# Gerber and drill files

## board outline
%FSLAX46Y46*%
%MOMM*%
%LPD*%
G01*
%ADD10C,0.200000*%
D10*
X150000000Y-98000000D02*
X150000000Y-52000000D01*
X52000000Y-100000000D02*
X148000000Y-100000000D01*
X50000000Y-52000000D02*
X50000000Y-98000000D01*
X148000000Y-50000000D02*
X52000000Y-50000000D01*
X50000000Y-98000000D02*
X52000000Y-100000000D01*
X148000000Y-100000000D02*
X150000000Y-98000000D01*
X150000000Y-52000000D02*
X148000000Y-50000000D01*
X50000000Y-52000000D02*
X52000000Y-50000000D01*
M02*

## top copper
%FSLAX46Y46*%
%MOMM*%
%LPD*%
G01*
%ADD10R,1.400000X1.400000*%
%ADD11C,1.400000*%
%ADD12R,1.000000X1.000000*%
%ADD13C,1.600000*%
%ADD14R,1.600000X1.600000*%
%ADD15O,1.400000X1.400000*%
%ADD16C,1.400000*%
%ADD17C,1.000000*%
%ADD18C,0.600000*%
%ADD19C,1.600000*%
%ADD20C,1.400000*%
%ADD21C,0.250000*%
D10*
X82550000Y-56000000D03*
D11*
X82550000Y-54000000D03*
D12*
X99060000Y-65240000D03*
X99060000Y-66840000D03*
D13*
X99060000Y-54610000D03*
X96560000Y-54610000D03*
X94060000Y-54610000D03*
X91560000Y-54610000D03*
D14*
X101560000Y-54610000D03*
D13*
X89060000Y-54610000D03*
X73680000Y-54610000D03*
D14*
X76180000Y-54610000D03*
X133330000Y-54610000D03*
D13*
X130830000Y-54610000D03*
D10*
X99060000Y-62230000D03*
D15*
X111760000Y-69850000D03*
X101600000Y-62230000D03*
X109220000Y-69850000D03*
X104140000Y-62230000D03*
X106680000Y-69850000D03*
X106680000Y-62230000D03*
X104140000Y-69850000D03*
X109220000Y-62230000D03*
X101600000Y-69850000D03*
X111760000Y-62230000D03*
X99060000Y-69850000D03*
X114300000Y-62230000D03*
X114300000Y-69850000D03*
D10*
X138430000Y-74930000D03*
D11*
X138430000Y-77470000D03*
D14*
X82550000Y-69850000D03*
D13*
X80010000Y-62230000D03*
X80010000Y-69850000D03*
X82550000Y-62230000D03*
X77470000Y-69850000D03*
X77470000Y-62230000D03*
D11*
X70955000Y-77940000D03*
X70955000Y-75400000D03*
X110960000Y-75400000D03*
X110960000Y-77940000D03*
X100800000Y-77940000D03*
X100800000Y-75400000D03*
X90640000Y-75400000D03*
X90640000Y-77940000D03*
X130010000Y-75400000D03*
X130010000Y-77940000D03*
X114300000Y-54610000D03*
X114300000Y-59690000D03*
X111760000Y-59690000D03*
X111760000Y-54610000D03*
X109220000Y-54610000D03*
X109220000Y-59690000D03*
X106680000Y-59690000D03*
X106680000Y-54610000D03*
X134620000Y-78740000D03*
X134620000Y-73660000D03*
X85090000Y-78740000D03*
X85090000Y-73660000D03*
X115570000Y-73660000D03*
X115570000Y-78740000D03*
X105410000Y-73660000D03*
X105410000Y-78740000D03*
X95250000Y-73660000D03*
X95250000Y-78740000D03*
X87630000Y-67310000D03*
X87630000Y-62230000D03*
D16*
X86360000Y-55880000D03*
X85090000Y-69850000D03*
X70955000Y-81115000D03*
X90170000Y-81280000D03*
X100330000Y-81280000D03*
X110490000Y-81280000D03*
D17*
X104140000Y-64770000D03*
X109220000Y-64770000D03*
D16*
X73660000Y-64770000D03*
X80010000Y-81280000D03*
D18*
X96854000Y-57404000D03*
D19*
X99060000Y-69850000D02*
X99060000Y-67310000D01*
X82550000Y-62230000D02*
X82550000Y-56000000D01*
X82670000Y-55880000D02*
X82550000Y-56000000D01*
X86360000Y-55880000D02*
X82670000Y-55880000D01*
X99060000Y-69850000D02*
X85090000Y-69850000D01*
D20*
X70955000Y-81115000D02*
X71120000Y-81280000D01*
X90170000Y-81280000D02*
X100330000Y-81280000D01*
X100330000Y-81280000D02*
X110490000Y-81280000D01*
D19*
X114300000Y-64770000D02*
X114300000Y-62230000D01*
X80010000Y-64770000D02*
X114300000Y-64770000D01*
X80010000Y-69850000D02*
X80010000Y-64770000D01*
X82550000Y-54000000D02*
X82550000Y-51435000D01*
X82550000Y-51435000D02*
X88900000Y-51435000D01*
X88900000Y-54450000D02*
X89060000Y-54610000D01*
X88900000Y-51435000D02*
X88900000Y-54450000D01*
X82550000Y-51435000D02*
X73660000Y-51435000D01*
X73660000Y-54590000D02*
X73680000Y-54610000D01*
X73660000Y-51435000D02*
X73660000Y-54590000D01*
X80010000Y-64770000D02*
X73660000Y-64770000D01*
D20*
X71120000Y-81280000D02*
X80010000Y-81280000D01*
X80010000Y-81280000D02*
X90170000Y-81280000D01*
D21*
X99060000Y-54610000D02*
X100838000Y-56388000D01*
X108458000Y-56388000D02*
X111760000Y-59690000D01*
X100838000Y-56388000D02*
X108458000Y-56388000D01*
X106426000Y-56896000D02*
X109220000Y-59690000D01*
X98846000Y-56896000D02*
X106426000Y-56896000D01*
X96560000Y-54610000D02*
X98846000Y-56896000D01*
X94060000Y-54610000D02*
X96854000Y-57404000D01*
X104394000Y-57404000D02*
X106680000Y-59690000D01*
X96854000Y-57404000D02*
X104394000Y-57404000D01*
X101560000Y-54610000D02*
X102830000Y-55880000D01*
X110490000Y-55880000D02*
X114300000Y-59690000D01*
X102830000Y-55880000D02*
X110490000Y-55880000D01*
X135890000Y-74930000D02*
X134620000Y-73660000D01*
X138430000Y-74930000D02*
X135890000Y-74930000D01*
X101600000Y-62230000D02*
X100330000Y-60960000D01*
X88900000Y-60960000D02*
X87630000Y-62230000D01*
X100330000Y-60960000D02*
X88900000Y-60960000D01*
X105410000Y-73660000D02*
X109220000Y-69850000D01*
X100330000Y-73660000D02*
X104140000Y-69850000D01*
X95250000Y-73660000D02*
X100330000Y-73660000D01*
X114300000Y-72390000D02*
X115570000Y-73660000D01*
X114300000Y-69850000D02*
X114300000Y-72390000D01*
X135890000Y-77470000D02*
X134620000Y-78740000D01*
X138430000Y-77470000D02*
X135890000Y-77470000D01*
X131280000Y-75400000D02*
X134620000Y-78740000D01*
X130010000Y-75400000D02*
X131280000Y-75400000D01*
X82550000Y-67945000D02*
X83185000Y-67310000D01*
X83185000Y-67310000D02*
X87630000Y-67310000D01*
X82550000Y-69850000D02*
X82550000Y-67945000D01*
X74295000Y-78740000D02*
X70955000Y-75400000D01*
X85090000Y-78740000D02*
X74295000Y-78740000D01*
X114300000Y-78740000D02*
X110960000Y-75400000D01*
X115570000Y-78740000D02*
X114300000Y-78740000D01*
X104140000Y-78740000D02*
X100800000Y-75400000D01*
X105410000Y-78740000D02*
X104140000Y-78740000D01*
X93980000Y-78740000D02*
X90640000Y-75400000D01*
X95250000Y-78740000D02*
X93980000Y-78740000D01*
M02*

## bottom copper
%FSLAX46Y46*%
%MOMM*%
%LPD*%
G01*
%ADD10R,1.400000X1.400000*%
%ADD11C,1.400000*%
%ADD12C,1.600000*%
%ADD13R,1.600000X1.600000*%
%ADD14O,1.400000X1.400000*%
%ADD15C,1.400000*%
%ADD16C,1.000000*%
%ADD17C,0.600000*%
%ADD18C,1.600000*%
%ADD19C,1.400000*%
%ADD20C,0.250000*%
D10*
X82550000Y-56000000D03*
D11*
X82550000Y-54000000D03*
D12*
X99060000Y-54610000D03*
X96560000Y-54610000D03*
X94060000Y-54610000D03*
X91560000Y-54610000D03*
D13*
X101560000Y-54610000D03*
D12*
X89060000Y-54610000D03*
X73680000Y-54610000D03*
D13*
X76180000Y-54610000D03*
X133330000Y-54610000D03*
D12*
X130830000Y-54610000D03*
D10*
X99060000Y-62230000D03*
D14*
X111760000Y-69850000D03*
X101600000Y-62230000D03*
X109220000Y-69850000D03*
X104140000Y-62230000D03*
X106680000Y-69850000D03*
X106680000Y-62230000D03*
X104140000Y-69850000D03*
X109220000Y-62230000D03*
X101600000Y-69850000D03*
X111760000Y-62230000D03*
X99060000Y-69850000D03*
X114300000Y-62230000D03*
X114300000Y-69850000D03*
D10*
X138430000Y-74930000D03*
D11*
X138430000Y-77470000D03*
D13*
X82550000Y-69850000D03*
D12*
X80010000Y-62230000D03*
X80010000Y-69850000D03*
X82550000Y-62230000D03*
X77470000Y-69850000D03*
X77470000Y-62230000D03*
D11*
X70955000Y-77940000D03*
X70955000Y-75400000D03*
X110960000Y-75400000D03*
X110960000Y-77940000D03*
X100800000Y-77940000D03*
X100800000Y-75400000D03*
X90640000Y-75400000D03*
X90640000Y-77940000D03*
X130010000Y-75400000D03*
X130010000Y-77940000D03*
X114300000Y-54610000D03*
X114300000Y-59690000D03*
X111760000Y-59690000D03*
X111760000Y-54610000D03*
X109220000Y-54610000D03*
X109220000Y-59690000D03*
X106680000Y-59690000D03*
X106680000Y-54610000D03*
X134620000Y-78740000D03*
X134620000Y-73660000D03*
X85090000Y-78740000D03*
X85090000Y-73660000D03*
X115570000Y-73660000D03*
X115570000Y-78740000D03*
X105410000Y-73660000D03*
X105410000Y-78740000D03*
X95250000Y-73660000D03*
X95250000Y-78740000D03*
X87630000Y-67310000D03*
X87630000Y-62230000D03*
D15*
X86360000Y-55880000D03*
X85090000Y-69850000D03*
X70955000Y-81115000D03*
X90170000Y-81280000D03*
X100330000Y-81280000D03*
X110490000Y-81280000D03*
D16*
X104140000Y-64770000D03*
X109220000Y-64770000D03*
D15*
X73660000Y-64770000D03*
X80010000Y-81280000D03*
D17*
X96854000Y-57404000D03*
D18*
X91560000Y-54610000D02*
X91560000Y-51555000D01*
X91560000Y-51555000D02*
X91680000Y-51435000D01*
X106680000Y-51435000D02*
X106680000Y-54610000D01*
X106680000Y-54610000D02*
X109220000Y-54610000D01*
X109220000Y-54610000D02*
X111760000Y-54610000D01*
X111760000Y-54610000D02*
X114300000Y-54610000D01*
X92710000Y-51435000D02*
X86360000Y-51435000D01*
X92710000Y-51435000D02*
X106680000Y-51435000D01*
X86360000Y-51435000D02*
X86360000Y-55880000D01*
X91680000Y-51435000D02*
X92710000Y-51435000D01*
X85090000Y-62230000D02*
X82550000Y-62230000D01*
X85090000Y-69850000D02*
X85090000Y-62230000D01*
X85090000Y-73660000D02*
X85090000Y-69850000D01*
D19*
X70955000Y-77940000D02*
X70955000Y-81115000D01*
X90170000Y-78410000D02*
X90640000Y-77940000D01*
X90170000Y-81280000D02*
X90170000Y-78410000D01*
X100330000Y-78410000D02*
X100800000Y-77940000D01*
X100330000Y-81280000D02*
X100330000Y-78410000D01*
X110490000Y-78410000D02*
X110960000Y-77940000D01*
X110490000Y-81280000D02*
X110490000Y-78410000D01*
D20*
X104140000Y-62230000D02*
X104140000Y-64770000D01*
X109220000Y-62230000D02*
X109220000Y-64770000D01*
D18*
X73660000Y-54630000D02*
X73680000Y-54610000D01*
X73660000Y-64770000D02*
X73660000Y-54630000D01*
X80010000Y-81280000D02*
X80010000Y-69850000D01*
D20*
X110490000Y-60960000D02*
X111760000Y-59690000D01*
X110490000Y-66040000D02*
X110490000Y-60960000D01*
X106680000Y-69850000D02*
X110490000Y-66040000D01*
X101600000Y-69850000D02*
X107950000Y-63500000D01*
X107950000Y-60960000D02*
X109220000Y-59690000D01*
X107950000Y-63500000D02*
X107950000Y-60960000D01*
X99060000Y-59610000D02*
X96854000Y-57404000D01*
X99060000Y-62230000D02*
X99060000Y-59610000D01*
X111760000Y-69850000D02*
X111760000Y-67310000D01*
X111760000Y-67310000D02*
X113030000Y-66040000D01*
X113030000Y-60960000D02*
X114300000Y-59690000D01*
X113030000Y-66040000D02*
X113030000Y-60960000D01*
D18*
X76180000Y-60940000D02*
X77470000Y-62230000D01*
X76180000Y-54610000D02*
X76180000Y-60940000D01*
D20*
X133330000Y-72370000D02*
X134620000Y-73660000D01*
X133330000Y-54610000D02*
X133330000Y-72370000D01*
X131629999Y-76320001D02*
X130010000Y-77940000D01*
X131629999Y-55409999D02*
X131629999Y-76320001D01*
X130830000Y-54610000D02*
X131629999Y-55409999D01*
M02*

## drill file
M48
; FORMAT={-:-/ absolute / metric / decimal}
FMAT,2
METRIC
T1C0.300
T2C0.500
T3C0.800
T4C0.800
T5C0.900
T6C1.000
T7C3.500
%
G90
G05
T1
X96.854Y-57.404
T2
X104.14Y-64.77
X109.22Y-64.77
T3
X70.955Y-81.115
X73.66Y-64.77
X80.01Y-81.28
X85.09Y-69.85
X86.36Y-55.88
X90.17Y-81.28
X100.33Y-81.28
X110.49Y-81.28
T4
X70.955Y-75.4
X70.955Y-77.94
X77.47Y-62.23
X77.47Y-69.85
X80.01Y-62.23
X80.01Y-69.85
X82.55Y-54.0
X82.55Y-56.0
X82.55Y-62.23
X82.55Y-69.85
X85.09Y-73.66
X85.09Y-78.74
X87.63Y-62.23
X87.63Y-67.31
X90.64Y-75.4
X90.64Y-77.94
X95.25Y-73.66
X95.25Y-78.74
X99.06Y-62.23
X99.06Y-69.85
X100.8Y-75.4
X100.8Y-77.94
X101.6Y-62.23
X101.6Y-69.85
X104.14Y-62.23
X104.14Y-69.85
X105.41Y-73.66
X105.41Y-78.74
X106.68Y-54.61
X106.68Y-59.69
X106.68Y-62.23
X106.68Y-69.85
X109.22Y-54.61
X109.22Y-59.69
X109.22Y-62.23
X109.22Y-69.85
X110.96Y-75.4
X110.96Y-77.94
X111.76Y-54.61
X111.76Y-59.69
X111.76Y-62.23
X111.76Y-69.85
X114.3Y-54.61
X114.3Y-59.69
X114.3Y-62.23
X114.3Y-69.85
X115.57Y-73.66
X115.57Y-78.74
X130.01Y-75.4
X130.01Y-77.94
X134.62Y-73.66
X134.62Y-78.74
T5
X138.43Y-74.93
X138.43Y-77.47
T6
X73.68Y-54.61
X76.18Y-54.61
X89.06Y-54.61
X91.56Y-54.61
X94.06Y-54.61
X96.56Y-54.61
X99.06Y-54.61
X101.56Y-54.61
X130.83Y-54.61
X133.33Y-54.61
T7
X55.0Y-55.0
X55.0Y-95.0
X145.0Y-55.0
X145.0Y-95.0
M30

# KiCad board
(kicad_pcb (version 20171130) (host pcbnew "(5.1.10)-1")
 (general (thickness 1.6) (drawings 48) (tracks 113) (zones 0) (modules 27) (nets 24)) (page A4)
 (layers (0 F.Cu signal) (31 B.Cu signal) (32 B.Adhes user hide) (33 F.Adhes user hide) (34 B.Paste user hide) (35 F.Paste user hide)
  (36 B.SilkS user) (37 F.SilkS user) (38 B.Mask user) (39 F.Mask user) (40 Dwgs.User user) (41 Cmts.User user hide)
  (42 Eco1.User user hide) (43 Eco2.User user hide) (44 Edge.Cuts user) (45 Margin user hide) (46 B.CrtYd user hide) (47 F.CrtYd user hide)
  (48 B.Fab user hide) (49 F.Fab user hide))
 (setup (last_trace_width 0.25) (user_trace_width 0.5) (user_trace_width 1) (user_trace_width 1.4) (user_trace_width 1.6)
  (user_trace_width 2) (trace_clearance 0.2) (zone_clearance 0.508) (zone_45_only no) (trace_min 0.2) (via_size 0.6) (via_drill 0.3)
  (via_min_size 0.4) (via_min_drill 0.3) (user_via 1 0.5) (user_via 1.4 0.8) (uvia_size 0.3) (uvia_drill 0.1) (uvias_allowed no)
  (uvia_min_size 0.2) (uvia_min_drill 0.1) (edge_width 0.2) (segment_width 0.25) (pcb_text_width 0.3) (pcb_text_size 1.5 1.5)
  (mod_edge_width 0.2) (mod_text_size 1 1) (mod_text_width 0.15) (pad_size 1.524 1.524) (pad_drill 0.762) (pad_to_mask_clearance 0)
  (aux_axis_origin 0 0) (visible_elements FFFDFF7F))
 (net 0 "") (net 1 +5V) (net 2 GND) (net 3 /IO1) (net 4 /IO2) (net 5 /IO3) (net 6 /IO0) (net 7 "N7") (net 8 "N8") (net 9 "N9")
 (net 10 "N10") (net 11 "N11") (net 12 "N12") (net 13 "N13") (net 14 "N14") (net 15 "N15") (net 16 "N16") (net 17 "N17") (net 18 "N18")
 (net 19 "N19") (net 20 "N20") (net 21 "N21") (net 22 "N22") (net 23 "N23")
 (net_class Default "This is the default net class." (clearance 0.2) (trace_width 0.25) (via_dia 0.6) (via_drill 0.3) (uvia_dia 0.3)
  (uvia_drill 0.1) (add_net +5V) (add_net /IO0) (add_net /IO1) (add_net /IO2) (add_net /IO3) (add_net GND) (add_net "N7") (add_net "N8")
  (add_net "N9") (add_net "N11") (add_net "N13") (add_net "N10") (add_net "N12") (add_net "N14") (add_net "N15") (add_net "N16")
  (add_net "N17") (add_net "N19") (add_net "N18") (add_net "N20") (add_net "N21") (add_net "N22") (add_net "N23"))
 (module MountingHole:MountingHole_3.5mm (layer F.Cu) (at 145 55)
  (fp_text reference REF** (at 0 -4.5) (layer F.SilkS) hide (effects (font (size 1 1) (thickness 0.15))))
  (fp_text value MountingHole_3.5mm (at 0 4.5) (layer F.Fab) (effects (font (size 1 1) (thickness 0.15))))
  (pad 1 np_thru_hole circle (at 0 0) (size 3.5 3.5) (drill 3.5) (layers *.Cu *.Mask)))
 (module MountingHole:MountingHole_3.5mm (layer F.Cu) (at 145 95)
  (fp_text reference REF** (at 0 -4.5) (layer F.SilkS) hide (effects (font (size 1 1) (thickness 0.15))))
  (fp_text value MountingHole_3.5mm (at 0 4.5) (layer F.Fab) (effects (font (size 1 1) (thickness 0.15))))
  (pad 1 np_thru_hole circle (at 0 0) (size 3.5 3.5) (drill 3.5) (layers *.Cu *.Mask)))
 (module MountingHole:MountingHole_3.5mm (layer F.Cu) (at 55 95)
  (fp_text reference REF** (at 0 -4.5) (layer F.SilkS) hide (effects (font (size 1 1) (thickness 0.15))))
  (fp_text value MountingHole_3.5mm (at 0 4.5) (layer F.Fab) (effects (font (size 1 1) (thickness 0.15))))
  (pad 1 np_thru_hole circle (at 0 0) (size 3.5 3.5) (drill 3.5) (layers *.Cu *.Mask)))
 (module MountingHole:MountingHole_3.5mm (layer F.Cu) (at 55 55)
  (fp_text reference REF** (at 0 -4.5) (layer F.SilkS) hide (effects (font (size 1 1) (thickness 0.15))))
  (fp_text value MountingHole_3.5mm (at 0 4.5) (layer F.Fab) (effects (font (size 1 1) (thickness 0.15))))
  (pad 1 np_thru_hole circle (at 0 0) (size 3.5 3.5) (drill 3.5) (layers *.Cu *.Mask)))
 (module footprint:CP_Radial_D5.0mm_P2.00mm (layer B.Cu) (at 82.55 56 90)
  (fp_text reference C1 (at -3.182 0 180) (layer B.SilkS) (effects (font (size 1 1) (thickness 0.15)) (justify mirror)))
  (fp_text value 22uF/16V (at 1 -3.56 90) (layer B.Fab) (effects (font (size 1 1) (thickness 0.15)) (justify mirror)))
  (pad 1 thru_hole rect (at 0 0 90) (size 1.4 1.4) (drill 0.8) (layers *.Cu *.Mask) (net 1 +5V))
  (pad 2 thru_hole circle (at 2 0 90) (size 1.4 1.4) (drill 0.8) (layers *.Cu *.Mask) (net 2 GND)))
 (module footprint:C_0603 (layer F.Cu) (at 99.06 66.04 270)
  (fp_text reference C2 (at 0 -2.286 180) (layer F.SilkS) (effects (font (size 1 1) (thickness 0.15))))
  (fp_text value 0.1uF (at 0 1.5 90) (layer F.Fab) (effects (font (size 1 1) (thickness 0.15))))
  (pad 1 smd rect (at -0.8 0 270) (size 1 1) (layers F.Cu F.Paste F.Mask) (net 2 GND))
  (pad 2 smd rect (at 0.8 0 270) (size 1 1) (layers F.Cu F.Paste F.Mask) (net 1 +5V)))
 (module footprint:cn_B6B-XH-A (layer B.Cu) (at 95.31 54.61 180)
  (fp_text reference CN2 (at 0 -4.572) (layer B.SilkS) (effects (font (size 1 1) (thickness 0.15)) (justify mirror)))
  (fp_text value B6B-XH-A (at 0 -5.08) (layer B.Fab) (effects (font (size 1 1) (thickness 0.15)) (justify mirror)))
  (pad 2 thru_hole circle (at -3.75 0 180) (size 1.6 1.6) (drill 1) (layers *.Cu *.Mask) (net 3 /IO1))
  (pad 3 thru_hole circle (at -1.25 0 180) (size 1.6 1.6) (drill 1) (layers *.Cu *.Mask) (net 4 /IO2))
  (pad 4 thru_hole circle (at 1.25 0 180) (size 1.6 1.6) (drill 1) (layers *.Cu *.Mask) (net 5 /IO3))
  (pad 5 thru_hole circle (at 3.75 0 180) (size 1.6 1.6) (drill 1) (layers *.Cu *.Mask) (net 1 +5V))
  (pad 1 thru_hole rect (at -6.25 0 180) (size 1.6 1.6) (drill 1) (layers *.Cu *.Mask) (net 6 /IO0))
  (pad 6 thru_hole circle (at 6.25 0 180) (size 1.6 1.6) (drill 1) (layers *.Cu *.Mask) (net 2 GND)))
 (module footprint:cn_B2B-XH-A (layer B.Cu) (at 74.93 54.61 180)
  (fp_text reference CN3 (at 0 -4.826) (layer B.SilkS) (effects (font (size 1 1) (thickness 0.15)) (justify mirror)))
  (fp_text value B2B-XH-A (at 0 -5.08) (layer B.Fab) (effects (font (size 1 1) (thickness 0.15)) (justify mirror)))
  (pad 2 thru_hole circle (at 1.25 0 180) (size 1.6 1.6) (drill 1) (layers *.Cu *.Mask) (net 2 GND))
  (pad 1 thru_hole rect (at -1.25 0 180) (size 1.6 1.6) (drill 1) (layers *.Cu *.Mask) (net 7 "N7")))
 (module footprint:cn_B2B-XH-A (layer B.Cu) (at 132.08 54.61 180)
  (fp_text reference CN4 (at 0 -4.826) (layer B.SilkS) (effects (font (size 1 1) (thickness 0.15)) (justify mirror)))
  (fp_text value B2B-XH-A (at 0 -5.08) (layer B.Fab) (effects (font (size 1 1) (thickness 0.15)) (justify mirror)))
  (pad 1 thru_hole rect (at -1.25 0 180) (size 1.6 1.6) (drill 1) (layers *.Cu *.Mask) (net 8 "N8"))
  (pad 2 thru_hole circle (at 1.25 0 180) (size 1.6 1.6) (drill 1) (layers *.Cu *.Mask) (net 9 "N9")))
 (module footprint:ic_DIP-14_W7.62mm (layer B.Cu) (at 99.06 62.23 270)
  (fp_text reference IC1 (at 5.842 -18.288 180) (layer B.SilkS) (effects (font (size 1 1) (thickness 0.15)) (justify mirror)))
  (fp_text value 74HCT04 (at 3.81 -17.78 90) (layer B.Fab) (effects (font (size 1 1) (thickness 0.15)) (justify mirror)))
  (pad 1 thru_hole rect (at 0 0 270) (size 1.4 1.4) (drill 0.8) (layers *.Cu *.Mask) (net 5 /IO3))
  (pad 9 thru_hole oval (at 7.62 -12.7 270) (size 1.4 1.4) (drill 0.8) (layers *.Cu *.Mask) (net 6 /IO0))
  (pad 2 thru_hole oval (at 0 -2.54 270) (size 1.4 1.4) (drill 0.8) (layers *.Cu *.Mask) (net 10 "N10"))
  (pad 10 thru_hole oval (at 7.62 -10.16 270) (size 1.4 1.4) (drill 0.8) (layers *.Cu *.Mask) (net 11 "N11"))
  (pad 3 thru_hole oval (at 0 -5.08 270) (size 1.4 1.4) (drill 0.8) (layers *.Cu *.Mask) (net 2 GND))
  (pad 11 thru_hole oval (at 7.62 -7.62 270) (size 1.4 1.4) (drill 0.8) (layers *.Cu *.Mask) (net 3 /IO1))
  (pad 4 thru_hole oval (at 0 -7.62 270) (size 1.4 1.4) (drill 0.8) (layers *.Cu *.Mask) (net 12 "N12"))
  (pad 12 thru_hole oval (at 7.62 -5.08 270) (size 1.4 1.4) (drill 0.8) (layers *.Cu *.Mask) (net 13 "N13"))
  (pad 5 thru_hole oval (at 0 -10.16 270) (size 1.4 1.4) (drill 0.8) (layers *.Cu *.Mask) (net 2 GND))
  (pad 13 thru_hole oval (at 7.62 -2.54 270) (size 1.4 1.4) (drill 0.8) (layers *.Cu *.Mask) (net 4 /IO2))
  (pad 6 thru_hole oval (at 0 -12.7 270) (size 1.4 1.4) (drill 0.8) (layers *.Cu *.Mask) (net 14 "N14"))
  (pad 14 thru_hole oval (at 7.62 0 270) (size 1.4 1.4) (drill 0.8) (layers *.Cu *.Mask) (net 1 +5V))
  (pad 7 thru_hole oval (at 0 -15.24 270) (size 1.4 1.4) (drill 0.8) (layers *.Cu *.Mask) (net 2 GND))
  (pad 8 thru_hole oval (at 7.62 -15.24 270) (size 1.4 1.4) (drill 0.8) (layers *.Cu *.Mask) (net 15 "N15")))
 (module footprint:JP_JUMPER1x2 (layer B.Cu) (at 138.43 76.2 270)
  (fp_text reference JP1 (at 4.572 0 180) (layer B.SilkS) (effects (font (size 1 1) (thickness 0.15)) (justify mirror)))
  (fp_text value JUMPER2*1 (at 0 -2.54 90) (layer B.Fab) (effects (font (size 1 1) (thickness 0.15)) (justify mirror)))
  (pad 1 thru_hole rect (at -1.27 0 270) (size 1.4 1.4) (drill 0.9) (layers *.Cu *.Mask) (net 8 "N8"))
  (pad 2 thru_hole circle (at 1.27 0 270) (size 1.4 1.4) (drill 0.9) (layers *.Cu *.Mask) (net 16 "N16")))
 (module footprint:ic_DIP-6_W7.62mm (layer B.Cu) (at 82.55 69.85 90)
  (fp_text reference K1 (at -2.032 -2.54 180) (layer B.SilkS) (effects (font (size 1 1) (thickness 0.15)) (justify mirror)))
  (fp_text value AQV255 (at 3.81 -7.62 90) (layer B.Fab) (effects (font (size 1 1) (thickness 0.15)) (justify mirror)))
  (pad 1 thru_hole rect (at 0 0 90) (size 1.6 1.6) (drill 0.8) (layers *.Cu *.Mask) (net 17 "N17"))
  (pad 5 thru_hole circle (at 7.62 -2.54 90) (size 1.6 1.6) (drill 0.8) (layers *.Cu *.Mask) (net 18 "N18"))
  (pad 2 thru_hole circle (at 0 -2.54 90) (size 1.6 1.6) (drill 0.8) (layers *.Cu *.Mask) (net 2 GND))
  (pad 6 thru_hole circle (at 7.62 0 90) (size 1.6 1.6) (drill 0.8) (layers *.Cu *.Mask) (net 1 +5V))
  (pad 3 thru_hole circle (at 0 -5.08 90) (size 1.6 1.6) (drill 0.8) (layers *.Cu *.Mask) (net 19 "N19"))
  (pad 4 thru_hole circle (at 7.62 -5.08 90) (size 1.6 1.6) (drill 0.8) (layers *.Cu *.Mask) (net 7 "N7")))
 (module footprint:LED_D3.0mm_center (layer F.Cu) (at 70.955 76.67 270)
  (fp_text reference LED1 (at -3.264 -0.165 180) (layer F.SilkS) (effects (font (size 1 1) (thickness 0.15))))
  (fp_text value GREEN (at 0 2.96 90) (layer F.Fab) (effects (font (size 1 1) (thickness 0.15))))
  (pad 2 thru_hole circle (at 1.27 0 270) (size 1.4 1.4) (drill 0.8) (layers *.Cu *.Mask) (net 2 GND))
  (pad 1 thru_hole circle (at -1.27 0 270) (size 1.4 1.4) (drill 0.8) (layers *.Cu *.Mask) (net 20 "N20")))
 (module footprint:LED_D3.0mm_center (layer F.Cu) (at 110.96 76.67 270)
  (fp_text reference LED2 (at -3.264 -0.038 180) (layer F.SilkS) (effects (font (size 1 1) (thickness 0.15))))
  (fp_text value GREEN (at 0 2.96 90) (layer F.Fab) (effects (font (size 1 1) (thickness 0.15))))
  (pad 1 thru_hole circle (at -1.27 0 270) (size 1.4 1.4) (drill 0.8) (layers *.Cu *.Mask) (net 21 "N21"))
  (pad 2 thru_hole circle (at 1.27 0 270) (size 1.4 1.4) (drill 0.8) (layers *.Cu *.Mask) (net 2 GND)))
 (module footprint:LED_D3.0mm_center (layer F.Cu) (at 100.8 76.67 270)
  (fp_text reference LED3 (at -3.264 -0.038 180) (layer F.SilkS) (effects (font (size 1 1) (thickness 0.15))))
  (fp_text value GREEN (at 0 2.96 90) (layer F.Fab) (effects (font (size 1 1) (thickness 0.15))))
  (pad 2 thru_hole circle (at 1.27 0 270) (size 1.4 1.4) (drill 0.8) (layers *.Cu *.Mask) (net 2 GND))
  (pad 1 thru_hole circle (at -1.27 0 270) (size 1.4 1.4) (drill 0.8) (layers *.Cu *.Mask) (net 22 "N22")))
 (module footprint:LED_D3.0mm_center (layer F.Cu) (at 90.64 76.67 270)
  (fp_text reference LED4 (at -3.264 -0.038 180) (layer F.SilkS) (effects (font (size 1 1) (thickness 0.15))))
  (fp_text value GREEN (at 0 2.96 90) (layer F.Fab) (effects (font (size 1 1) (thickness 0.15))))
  (pad 1 thru_hole circle (at -1.27 0 270) (size 1.4 1.4) (drill 0.8) (layers *.Cu *.Mask) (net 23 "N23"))
  (pad 2 thru_hole circle (at 1.27 0 270) (size 1.4 1.4) (drill 0.8) (layers *.Cu *.Mask) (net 2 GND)))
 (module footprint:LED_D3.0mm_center (layer F.Cu) (at 130.01 76.67 270)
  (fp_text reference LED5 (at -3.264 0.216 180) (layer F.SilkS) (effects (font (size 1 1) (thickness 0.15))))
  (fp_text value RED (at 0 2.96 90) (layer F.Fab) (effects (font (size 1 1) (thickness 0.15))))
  (pad 1 thru_hole circle (at -1.27 0 270) (size 1.4 1.4) (drill 0.8) (layers *.Cu *.Mask) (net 16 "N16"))
  (pad 2 thru_hole circle (at 1.27 0 270) (size 1.4 1.4) (drill 0.8) (layers *.Cu *.Mask) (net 9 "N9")))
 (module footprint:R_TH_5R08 (layer B.Cu) (at 114.3 57.15 90)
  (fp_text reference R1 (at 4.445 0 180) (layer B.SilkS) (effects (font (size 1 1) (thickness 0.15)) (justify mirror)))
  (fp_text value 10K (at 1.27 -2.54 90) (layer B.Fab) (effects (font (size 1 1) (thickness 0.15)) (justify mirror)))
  (pad 2 thru_hole circle (at 2.54 0 90) (size 1.4 1.4) (drill 0.8) (layers *.Cu *.Mask) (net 1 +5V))
  (pad 1 thru_hole circle (at -2.54 0 90) (size 1.4 1.4) (drill 0.8) (layers *.Cu *.Mask) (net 6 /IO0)))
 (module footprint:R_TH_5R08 (layer B.Cu) (at 111.76 57.15 90)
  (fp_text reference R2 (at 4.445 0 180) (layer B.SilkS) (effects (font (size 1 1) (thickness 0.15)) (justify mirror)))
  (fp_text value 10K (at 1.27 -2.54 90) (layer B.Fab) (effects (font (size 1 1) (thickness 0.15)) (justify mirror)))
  (pad 1 thru_hole circle (at -2.54 0 90) (size 1.4 1.4) (drill 0.8) (layers *.Cu *.Mask) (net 3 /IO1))
  (pad 2 thru_hole circle (at 2.54 0 90) (size 1.4 1.4) (drill 0.8) (layers *.Cu *.Mask) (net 1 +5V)))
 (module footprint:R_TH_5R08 (layer B.Cu) (at 109.22 57.15 90)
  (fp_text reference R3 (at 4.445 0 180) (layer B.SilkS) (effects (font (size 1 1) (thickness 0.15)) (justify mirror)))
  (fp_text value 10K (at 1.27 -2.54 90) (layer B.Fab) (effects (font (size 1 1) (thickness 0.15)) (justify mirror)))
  (pad 2 thru_hole circle (at 2.54 0 90) (size 1.4 1.4) (drill 0.8) (layers *.Cu *.Mask) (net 1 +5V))
  (pad 1 thru_hole circle (at -2.54 0 90) (size 1.4 1.4) (drill 0.8) (layers *.Cu *.Mask) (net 4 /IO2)))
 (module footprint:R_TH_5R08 (layer B.Cu) (at 106.68 57.15 90)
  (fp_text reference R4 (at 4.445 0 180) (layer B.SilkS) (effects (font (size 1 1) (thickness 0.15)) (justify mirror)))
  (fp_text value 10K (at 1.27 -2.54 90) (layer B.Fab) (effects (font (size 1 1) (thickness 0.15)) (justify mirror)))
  (pad 1 thru_hole circle (at -2.54 0 90) (size 1.4 1.4) (drill 0.8) (layers *.Cu *.Mask) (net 5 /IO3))
  (pad 2 thru_hole circle (at 2.54 0 90) (size 1.4 1.4) (drill 0.8) (layers *.Cu *.Mask) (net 1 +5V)))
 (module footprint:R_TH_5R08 (layer B.Cu) (at 134.62 76.2 90)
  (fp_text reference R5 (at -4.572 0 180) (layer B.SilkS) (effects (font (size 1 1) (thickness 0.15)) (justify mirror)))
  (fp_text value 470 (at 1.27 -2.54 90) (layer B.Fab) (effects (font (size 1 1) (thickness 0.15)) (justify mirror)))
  (pad 1 thru_hole circle (at -2.54 0 90) (size 1.4 1.4) (drill 0.8) (layers *.Cu *.Mask) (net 16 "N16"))
  (pad 2 thru_hole circle (at 2.54 0 90) (size 1.4 1.4) (drill 0.8) (layers *.Cu *.Mask) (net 8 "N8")))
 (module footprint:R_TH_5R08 (layer B.Cu) (at 85.09 76.2 90)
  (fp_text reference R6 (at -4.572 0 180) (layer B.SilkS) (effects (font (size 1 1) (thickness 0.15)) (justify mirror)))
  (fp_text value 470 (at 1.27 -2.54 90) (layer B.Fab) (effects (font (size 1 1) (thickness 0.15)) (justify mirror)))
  (pad 1 thru_hole circle (at -2.54 0 90) (size 1.4 1.4) (drill 0.8) (layers *.Cu *.Mask) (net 20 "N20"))
  (pad 2 thru_hole circle (at 2.54 0 90) (size 1.4 1.4) (drill 0.8) (layers *.Cu *.Mask) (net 1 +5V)))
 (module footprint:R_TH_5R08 (layer B.Cu) (at 115.57 76.2 90)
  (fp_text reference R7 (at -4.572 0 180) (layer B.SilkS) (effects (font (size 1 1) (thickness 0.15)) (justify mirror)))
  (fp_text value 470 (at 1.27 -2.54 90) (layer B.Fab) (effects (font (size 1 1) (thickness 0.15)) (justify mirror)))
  (pad 2 thru_hole circle (at 2.54 0 90) (size 1.4 1.4) (drill 0.8) (layers *.Cu *.Mask) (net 15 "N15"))
  (pad 1 thru_hole circle (at -2.54 0 90) (size 1.4 1.4) (drill 0.8) (layers *.Cu *.Mask) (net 21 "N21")))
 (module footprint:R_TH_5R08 (layer B.Cu) (at 105.41 76.2 90)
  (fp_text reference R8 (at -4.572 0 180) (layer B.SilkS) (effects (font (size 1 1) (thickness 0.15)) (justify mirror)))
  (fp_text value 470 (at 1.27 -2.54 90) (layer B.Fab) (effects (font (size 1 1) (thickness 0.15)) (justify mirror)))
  (pad 2 thru_hole circle (at 2.54 0 90) (size 1.4 1.4) (drill 0.8) (layers *.Cu *.Mask) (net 11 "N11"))
  (pad 1 thru_hole circle (at -2.54 0 90) (size 1.4 1.4) (drill 0.8) (layers *.Cu *.Mask) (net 22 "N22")))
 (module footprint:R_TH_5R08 (layer B.Cu) (at 95.25 76.2 90)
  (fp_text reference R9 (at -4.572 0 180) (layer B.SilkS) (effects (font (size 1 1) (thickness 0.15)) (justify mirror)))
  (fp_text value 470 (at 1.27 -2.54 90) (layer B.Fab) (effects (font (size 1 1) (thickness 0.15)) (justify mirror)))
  (pad 2 thru_hole circle (at 2.54 0 90) (size 1.4 1.4) (drill 0.8) (layers *.Cu *.Mask) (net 13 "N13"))
  (pad 1 thru_hole circle (at -2.54 0 90) (size 1.4 1.4) (drill 0.8) (layers *.Cu *.Mask) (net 23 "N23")))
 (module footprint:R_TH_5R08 (layer B.Cu) (at 87.63 64.77 90)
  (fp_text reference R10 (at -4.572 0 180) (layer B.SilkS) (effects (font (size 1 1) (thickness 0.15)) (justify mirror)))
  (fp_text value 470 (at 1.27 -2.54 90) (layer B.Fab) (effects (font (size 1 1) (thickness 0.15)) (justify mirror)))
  (pad 1 thru_hole circle (at -2.54 0 90) (size 1.4 1.4) (drill 0.8) (layers *.Cu *.Mask) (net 17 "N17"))
  (pad 2 thru_hole circle (at 2.54 0 90) (size 1.4 1.4) (drill 0.8) (layers *.Cu *.Mask) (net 10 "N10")))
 (gr_line (start 150 98) (end 150 52) (layer Edge.Cuts) (width 0.2))
 (gr_line (start 52 100) (end 148 100) (layer Edge.Cuts) (width 0.2))
 (gr_line (start 50 52) (end 50 98) (layer Edge.Cuts) (width 0.2))
 (gr_line (start 148 50) (end 52 50) (layer Edge.Cuts) (width 0.2))
 (gr_line (start 50 98) (end 52 100) (layer Edge.Cuts) (width 0.2))
 (gr_line (start 148 100) (end 150 98) (layer Edge.Cuts) (width 0.2))
 (gr_line (start 150 52) (end 148 50) (layer Edge.Cuts) (width 0.2))
 (gr_line (start 50 52) (end 52 50) (layer Edge.Cuts) (width 0.2))
 (segment (start 99.06 69.85) (end 99.06 67.31) (width 1.6) (layer F.Cu) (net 1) (status 30))
 (segment (start 82.55 62.23) (end 82.55 56) (width 1.6) (layer F.Cu) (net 1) (status 30))
 (segment (start 91.56 54.61) (end 91.56 51.555) (width 1.6) (layer B.Cu) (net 1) (status 10))
 (segment (start 91.56 51.555) (end 91.68 51.435) (width 1.6) (layer B.Cu) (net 1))
 (segment (start 106.68 51.435) (end 106.68 54.61) (width 1.6) (layer B.Cu) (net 1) (status 20))
 (segment (start 106.68 54.61) (end 109.22 54.61) (width 1.6) (layer B.Cu) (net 1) (status 30))
 (segment (start 109.22 54.61) (end 111.76 54.61) (width 1.6) (layer B.Cu) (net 1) (status 30))
 (segment (start 111.76 54.61) (end 114.3 54.61) (width 1.6) (layer B.Cu) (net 1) (status 30))
 (segment (start 92.71 51.435) (end 86.36 51.435) (width 1.6) (layer B.Cu) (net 1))
 (segment (start 92.71 51.435) (end 106.68 51.435) (width 1.6) (layer B.Cu) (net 1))
 (via (at 86.36 55.88) (size 1.4) (drill 0.8) (layers F.Cu B.Cu) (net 1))
 (segment (start 86.36 51.435) (end 86.36 55.88) (width 1.6) (layer B.Cu) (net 1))
 (segment (start 82.67 55.88) (end 82.55 56) (width 1.6) (layer F.Cu) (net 1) (status 30))
 (segment (start 86.36 55.88) (end 82.67 55.88) (width 1.6) (layer F.Cu) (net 1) (status 20))
 (segment (start 91.68 51.435) (end 92.71 51.435) (width 1.6) (layer B.Cu) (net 1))
 (segment (start 85.09 62.23) (end 82.55 62.23) (width 1.6) (layer B.Cu) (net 1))
 (via (at 85.09 69.85) (size 1.4) (drill 0.8) (layers F.Cu B.Cu) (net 1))
 (segment (start 99.06 69.85) (end 85.09 69.85) (width 1.6) (layer F.Cu) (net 1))
 (segment (start 85.09 69.85) (end 85.09 62.23) (width 1.6) (layer B.Cu) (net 1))
 (segment (start 85.09 73.66) (end 85.09 69.85) (width 1.6) (layer B.Cu) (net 1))
 (segment (start 70.955 77.94) (end 70.955 81.115) (width 1.4) (layer B.Cu) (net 2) (status 10))
 (via (at 70.955 81.115) (size 1.4) (drill 0.8) (layers F.Cu B.Cu) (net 2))
 (via (at 90.17 81.28) (size 1.4) (drill 0.8) (layers F.Cu B.Cu) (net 2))
 (segment (start 90.17 78.41) (end 90.64 77.94) (width 1.4) (layer B.Cu) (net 2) (status 30))
 (segment (start 90.17 81.28) (end 90.17 78.41) (width 1.4) (layer B.Cu) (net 2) (status 20))
 (segment (start 70.955 81.115) (end 71.12 81.28) (width 1.4) (layer F.Cu) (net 2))
 (via (at 100.33 81.28) (size 1.4) (drill 0.8) (layers F.Cu B.Cu) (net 2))
 (segment (start 90.17 81.28) (end 100.33 81.28) (width 1.4) (layer F.Cu) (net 2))
 (segment (start 100.33 78.41) (end 100.8 77.94) (width 1.4) (layer B.Cu) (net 2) (status 30))
 (segment (start 100.33 81.28) (end 100.33 78.41) (width 1.4) (layer B.Cu) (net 2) (status 20))
 (segment (start 100.33 81.28) (end 110.49 81.28) (width 1.4) (layer F.Cu) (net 2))
 (via (at 110.49 81.28) (size 1.4) (drill 0.8) (layers F.Cu B.Cu) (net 2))
 (segment (start 110.49 78.41) (end 110.96 77.94) (width 1.4) (layer B.Cu) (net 2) (status 30))
 (segment (start 110.49 81.28) (end 110.49 78.41) (width 1.4) (layer B.Cu) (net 2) (status 20))
 (segment (start 104.14 62.23) (end 104.14 64.77) (width 0.25) (layer B.Cu) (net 2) (status 10))
 (via (at 104.14 64.77) (size 1) (drill 0.5) (layers F.Cu B.Cu) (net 2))
 (segment (start 109.22 62.23) (end 109.22 64.77) (width 0.25) (layer B.Cu) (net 2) (status 10))
 (via (at 109.22 64.77) (size 1) (drill 0.5) (layers F.Cu B.Cu) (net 2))
 (segment (start 114.3 64.77) (end 114.3 62.23) (width 1.6) (layer F.Cu) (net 2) (status 20))
 (segment (start 80.01 64.77) (end 114.3 64.77) (width 1.6) (layer F.Cu) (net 2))
 (segment (start 80.01 69.85) (end 80.01 64.77) (width 1.6) (layer F.Cu) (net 2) (status 10))
 (segment (start 82.55 54) (end 82.55 51.435) (width 1.6) (layer F.Cu) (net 2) (status 10))
 (segment (start 82.55 51.435) (end 88.9 51.435) (width 1.6) (layer F.Cu) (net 2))
 (segment (start 88.9 54.45) (end 89.06 54.61) (width 1.6) (layer F.Cu) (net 2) (status 30))
 (segment (start 88.9 51.435) (end 88.9 54.45) (width 1.6) (layer F.Cu) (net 2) (status 20))
 (segment (start 82.55 51.435) (end 73.66 51.435) (width 1.6) (layer F.Cu) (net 2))
 (segment (start 73.66 54.59) (end 73.68 54.61) (width 1.6) (layer F.Cu) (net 2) (status 30))
 (segment (start 73.66 51.435) (end 73.66 54.59) (width 1.6) (layer F.Cu) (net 2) (status 20))
 (segment (start 80.01 64.77) (end 73.66 64.77) (width 1.6) (layer F.Cu) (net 2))
 (via (at 73.66 64.77) (size 1.4) (drill 0.8) (layers F.Cu B.Cu) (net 2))
 (segment (start 73.66 54.63) (end 73.68 54.61) (width 1.6) (layer B.Cu) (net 2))
 (segment (start 73.66 64.77) (end 73.66 54.63) (width 1.6) (layer B.Cu) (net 2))
 (via (at 80.01 81.28) (size 1.4) (drill 0.8) (layers F.Cu B.Cu) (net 2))
 (segment (start 71.12 81.28) (end 80.01 81.28) (width 1.4) (layer F.Cu) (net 2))
 (segment (start 80.01 81.28) (end 90.17 81.28) (width 1.4) (layer F.Cu) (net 2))
 (segment (start 80.01 81.28) (end 80.01 69.85) (width 1.6) (layer B.Cu) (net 2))
 (segment (start 99.06 54.61) (end 100.838 56.388) (width 0.25) (layer F.Cu) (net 3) (status 10))
 (segment (start 108.458 56.388) (end 111.76 59.69) (width 0.25) (layer F.Cu) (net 3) (status 20))
 (segment (start 100.838 56.388) (end 108.458 56.388) (width 0.25) (layer F.Cu) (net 3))
 (segment (start 110.49 60.96) (end 111.76 59.69) (width 0.25) (layer B.Cu) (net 3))
 (segment (start 110.49 66.04) (end 110.49 60.96) (width 0.25) (layer B.Cu) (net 3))
 (segment (start 106.68 69.85) (end 110.49 66.04) (width 0.25) (layer B.Cu) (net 3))
 (segment (start 106.426 56.896) (end 109.22 59.69) (width 0.25) (layer F.Cu) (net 4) (status 20))
 (segment (start 98.846 56.896) (end 106.426 56.896) (width 0.25) (layer F.Cu) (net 4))
 (segment (start 96.56 54.61) (end 98.846 56.896) (width 0.25) (layer F.Cu) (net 4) (status 10))
 (segment (start 101.6 69.85) (end 107.95 63.5) (width 0.25) (layer B.Cu) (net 4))
 (segment (start 107.95 60.96) (end 109.22 59.69) (width 0.25) (layer B.Cu) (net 4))
 (segment (start 107.95 63.5) (end 107.95 60.96) (width 0.25) (layer B.Cu) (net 4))
 (segment (start 94.06 54.61) (end 96.854 57.404) (width 0.25) (layer F.Cu) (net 5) (status 10))
 (segment (start 104.394 57.404) (end 106.68 59.69) (width 0.25) (layer F.Cu) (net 5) (status 20))
 (segment (start 96.854 57.404) (end 104.394 57.404) (width 0.25) (layer F.Cu) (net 5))
 (via (at 96.854 57.404) (size 0.6) (drill 0.3) (layers F.Cu B.Cu) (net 5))
 (segment (start 99.06 59.61) (end 96.854 57.404) (width 0.25) (layer B.Cu) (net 5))
 (segment (start 99.06 62.23) (end 99.06 59.61) (width 0.25) (layer B.Cu) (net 5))
 (segment (start 101.56 54.61) (end 102.83 55.88) (width 0.25) (layer F.Cu) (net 6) (status 10))
 (segment (start 110.49 55.88) (end 114.3 59.69) (width 0.25) (layer F.Cu) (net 6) (status 20))
 (segment (start 102.83 55.88) (end 110.49 55.88) (width 0.25) (layer F.Cu) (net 6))
 (segment (start 111.76 69.85) (end 111.76 67.31) (width 0.25) (layer B.Cu) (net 6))
 (segment (start 111.76 67.31) (end 113.03 66.04) (width 0.25) (layer B.Cu) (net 6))
 (segment (start 113.03 60.96) (end 114.3 59.69) (width 0.25) (layer B.Cu) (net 6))
 (segment (start 113.03 66.04) (end 113.03 60.96) (width 0.25) (layer B.Cu) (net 6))
 (segment (start 76.18 60.94) (end 77.47 62.23) (width 1.6) (layer B.Cu) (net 7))
 (segment (start 76.18 54.61) (end 76.18 60.94) (width 1.6) (layer B.Cu) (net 7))
 (segment (start 135.89 74.93) (end 134.62 73.66) (width 0.25) (layer F.Cu) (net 8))
 (segment (start 138.43 74.93) (end 135.89 74.93) (width 0.25) (layer F.Cu) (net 8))
 (segment (start 133.33 72.37) (end 134.62 73.66) (width 0.25) (layer B.Cu) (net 8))
 (segment (start 133.33 54.61) (end 133.33 72.37) (width 0.25) (layer B.Cu) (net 8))
 (segment (start 131.629999 76.320001) (end 130.01 77.94) (width 0.25) (layer B.Cu) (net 9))
 (segment (start 131.629999 55.409999) (end 131.629999 76.320001) (width 0.25) (layer B.Cu) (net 9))
 (segment (start 130.83 54.61) (end 131.629999 55.409999) (width 0.25) (layer B.Cu) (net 9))
 (segment (start 101.6 62.23) (end 100.33 60.96) (width 0.25) (layer F.Cu) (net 10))
 (segment (start 88.9 60.96) (end 87.63 62.23) (width 0.25) (layer F.Cu) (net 10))
 (segment (start 100.33 60.96) (end 88.9 60.96) (width 0.25) (layer F.Cu) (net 10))
 (segment (start 105.41 73.66) (end 109.22 69.85) (width 0.25) (layer F.Cu) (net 11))
 (segment (start 100.33 73.66) (end 104.14 69.85) (width 0.25) (layer F.Cu) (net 13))
 (segment (start 95.25 73.66) (end 100.33 73.66) (width 0.25) (layer F.Cu) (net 13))
 (segment (start 114.3 72.39) (end 115.57 73.66) (width 0.25) (layer F.Cu) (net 15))
 (segment (start 114.3 69.85) (end 114.3 72.39) (width 0.25) (layer F.Cu) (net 15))
 (segment (start 135.89 77.47) (end 134.62 78.74) (width 0.25) (layer F.Cu) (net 16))
 (segment (start 138.43 77.47) (end 135.89 77.47) (width 0.25) (layer F.Cu) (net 16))
 (segment (start 131.28 75.4) (end 134.62 78.74) (width 0.25) (layer F.Cu) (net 16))
 (segment (start 130.01 75.4) (end 131.28 75.4) (width 0.25) (layer F.Cu) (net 16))
 (segment (start 82.55 67.945) (end 83.185 67.31) (width 0.25) (layer F.Cu) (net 17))
 (segment (start 83.185 67.31) (end 87.63 67.31) (width 0.25) (layer F.Cu) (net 17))
 (segment (start 82.55 69.85) (end 82.55 67.945) (width 0.25) (layer F.Cu) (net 17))
 (segment (start 74.295 78.74) (end 70.955 75.4) (width 0.25) (layer F.Cu) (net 20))
 (segment (start 85.09 78.74) (end 74.295 78.74) (width 0.25) (layer F.Cu) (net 20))
 (segment (start 114.3 78.74) (end 110.96 75.4) (width 0.25) (layer F.Cu) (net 21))
 (segment (start 115.57 78.74) (end 114.3 78.74) (width 0.25) (layer F.Cu) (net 21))
 (segment (start 104.14 78.74) (end 100.8 75.4) (width 0.25) (layer F.Cu) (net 22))
 (segment (start 105.41 78.74) (end 104.14 78.74) (width 0.25) (layer F.Cu) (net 22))
 (segment (start 93.98 78.74) (end 90.64 75.4) (width 0.25) (layer F.Cu) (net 23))
 (segment (start 95.25 78.74) (end 93.98 78.74) (width 0.25) (layer F.Cu) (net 23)))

